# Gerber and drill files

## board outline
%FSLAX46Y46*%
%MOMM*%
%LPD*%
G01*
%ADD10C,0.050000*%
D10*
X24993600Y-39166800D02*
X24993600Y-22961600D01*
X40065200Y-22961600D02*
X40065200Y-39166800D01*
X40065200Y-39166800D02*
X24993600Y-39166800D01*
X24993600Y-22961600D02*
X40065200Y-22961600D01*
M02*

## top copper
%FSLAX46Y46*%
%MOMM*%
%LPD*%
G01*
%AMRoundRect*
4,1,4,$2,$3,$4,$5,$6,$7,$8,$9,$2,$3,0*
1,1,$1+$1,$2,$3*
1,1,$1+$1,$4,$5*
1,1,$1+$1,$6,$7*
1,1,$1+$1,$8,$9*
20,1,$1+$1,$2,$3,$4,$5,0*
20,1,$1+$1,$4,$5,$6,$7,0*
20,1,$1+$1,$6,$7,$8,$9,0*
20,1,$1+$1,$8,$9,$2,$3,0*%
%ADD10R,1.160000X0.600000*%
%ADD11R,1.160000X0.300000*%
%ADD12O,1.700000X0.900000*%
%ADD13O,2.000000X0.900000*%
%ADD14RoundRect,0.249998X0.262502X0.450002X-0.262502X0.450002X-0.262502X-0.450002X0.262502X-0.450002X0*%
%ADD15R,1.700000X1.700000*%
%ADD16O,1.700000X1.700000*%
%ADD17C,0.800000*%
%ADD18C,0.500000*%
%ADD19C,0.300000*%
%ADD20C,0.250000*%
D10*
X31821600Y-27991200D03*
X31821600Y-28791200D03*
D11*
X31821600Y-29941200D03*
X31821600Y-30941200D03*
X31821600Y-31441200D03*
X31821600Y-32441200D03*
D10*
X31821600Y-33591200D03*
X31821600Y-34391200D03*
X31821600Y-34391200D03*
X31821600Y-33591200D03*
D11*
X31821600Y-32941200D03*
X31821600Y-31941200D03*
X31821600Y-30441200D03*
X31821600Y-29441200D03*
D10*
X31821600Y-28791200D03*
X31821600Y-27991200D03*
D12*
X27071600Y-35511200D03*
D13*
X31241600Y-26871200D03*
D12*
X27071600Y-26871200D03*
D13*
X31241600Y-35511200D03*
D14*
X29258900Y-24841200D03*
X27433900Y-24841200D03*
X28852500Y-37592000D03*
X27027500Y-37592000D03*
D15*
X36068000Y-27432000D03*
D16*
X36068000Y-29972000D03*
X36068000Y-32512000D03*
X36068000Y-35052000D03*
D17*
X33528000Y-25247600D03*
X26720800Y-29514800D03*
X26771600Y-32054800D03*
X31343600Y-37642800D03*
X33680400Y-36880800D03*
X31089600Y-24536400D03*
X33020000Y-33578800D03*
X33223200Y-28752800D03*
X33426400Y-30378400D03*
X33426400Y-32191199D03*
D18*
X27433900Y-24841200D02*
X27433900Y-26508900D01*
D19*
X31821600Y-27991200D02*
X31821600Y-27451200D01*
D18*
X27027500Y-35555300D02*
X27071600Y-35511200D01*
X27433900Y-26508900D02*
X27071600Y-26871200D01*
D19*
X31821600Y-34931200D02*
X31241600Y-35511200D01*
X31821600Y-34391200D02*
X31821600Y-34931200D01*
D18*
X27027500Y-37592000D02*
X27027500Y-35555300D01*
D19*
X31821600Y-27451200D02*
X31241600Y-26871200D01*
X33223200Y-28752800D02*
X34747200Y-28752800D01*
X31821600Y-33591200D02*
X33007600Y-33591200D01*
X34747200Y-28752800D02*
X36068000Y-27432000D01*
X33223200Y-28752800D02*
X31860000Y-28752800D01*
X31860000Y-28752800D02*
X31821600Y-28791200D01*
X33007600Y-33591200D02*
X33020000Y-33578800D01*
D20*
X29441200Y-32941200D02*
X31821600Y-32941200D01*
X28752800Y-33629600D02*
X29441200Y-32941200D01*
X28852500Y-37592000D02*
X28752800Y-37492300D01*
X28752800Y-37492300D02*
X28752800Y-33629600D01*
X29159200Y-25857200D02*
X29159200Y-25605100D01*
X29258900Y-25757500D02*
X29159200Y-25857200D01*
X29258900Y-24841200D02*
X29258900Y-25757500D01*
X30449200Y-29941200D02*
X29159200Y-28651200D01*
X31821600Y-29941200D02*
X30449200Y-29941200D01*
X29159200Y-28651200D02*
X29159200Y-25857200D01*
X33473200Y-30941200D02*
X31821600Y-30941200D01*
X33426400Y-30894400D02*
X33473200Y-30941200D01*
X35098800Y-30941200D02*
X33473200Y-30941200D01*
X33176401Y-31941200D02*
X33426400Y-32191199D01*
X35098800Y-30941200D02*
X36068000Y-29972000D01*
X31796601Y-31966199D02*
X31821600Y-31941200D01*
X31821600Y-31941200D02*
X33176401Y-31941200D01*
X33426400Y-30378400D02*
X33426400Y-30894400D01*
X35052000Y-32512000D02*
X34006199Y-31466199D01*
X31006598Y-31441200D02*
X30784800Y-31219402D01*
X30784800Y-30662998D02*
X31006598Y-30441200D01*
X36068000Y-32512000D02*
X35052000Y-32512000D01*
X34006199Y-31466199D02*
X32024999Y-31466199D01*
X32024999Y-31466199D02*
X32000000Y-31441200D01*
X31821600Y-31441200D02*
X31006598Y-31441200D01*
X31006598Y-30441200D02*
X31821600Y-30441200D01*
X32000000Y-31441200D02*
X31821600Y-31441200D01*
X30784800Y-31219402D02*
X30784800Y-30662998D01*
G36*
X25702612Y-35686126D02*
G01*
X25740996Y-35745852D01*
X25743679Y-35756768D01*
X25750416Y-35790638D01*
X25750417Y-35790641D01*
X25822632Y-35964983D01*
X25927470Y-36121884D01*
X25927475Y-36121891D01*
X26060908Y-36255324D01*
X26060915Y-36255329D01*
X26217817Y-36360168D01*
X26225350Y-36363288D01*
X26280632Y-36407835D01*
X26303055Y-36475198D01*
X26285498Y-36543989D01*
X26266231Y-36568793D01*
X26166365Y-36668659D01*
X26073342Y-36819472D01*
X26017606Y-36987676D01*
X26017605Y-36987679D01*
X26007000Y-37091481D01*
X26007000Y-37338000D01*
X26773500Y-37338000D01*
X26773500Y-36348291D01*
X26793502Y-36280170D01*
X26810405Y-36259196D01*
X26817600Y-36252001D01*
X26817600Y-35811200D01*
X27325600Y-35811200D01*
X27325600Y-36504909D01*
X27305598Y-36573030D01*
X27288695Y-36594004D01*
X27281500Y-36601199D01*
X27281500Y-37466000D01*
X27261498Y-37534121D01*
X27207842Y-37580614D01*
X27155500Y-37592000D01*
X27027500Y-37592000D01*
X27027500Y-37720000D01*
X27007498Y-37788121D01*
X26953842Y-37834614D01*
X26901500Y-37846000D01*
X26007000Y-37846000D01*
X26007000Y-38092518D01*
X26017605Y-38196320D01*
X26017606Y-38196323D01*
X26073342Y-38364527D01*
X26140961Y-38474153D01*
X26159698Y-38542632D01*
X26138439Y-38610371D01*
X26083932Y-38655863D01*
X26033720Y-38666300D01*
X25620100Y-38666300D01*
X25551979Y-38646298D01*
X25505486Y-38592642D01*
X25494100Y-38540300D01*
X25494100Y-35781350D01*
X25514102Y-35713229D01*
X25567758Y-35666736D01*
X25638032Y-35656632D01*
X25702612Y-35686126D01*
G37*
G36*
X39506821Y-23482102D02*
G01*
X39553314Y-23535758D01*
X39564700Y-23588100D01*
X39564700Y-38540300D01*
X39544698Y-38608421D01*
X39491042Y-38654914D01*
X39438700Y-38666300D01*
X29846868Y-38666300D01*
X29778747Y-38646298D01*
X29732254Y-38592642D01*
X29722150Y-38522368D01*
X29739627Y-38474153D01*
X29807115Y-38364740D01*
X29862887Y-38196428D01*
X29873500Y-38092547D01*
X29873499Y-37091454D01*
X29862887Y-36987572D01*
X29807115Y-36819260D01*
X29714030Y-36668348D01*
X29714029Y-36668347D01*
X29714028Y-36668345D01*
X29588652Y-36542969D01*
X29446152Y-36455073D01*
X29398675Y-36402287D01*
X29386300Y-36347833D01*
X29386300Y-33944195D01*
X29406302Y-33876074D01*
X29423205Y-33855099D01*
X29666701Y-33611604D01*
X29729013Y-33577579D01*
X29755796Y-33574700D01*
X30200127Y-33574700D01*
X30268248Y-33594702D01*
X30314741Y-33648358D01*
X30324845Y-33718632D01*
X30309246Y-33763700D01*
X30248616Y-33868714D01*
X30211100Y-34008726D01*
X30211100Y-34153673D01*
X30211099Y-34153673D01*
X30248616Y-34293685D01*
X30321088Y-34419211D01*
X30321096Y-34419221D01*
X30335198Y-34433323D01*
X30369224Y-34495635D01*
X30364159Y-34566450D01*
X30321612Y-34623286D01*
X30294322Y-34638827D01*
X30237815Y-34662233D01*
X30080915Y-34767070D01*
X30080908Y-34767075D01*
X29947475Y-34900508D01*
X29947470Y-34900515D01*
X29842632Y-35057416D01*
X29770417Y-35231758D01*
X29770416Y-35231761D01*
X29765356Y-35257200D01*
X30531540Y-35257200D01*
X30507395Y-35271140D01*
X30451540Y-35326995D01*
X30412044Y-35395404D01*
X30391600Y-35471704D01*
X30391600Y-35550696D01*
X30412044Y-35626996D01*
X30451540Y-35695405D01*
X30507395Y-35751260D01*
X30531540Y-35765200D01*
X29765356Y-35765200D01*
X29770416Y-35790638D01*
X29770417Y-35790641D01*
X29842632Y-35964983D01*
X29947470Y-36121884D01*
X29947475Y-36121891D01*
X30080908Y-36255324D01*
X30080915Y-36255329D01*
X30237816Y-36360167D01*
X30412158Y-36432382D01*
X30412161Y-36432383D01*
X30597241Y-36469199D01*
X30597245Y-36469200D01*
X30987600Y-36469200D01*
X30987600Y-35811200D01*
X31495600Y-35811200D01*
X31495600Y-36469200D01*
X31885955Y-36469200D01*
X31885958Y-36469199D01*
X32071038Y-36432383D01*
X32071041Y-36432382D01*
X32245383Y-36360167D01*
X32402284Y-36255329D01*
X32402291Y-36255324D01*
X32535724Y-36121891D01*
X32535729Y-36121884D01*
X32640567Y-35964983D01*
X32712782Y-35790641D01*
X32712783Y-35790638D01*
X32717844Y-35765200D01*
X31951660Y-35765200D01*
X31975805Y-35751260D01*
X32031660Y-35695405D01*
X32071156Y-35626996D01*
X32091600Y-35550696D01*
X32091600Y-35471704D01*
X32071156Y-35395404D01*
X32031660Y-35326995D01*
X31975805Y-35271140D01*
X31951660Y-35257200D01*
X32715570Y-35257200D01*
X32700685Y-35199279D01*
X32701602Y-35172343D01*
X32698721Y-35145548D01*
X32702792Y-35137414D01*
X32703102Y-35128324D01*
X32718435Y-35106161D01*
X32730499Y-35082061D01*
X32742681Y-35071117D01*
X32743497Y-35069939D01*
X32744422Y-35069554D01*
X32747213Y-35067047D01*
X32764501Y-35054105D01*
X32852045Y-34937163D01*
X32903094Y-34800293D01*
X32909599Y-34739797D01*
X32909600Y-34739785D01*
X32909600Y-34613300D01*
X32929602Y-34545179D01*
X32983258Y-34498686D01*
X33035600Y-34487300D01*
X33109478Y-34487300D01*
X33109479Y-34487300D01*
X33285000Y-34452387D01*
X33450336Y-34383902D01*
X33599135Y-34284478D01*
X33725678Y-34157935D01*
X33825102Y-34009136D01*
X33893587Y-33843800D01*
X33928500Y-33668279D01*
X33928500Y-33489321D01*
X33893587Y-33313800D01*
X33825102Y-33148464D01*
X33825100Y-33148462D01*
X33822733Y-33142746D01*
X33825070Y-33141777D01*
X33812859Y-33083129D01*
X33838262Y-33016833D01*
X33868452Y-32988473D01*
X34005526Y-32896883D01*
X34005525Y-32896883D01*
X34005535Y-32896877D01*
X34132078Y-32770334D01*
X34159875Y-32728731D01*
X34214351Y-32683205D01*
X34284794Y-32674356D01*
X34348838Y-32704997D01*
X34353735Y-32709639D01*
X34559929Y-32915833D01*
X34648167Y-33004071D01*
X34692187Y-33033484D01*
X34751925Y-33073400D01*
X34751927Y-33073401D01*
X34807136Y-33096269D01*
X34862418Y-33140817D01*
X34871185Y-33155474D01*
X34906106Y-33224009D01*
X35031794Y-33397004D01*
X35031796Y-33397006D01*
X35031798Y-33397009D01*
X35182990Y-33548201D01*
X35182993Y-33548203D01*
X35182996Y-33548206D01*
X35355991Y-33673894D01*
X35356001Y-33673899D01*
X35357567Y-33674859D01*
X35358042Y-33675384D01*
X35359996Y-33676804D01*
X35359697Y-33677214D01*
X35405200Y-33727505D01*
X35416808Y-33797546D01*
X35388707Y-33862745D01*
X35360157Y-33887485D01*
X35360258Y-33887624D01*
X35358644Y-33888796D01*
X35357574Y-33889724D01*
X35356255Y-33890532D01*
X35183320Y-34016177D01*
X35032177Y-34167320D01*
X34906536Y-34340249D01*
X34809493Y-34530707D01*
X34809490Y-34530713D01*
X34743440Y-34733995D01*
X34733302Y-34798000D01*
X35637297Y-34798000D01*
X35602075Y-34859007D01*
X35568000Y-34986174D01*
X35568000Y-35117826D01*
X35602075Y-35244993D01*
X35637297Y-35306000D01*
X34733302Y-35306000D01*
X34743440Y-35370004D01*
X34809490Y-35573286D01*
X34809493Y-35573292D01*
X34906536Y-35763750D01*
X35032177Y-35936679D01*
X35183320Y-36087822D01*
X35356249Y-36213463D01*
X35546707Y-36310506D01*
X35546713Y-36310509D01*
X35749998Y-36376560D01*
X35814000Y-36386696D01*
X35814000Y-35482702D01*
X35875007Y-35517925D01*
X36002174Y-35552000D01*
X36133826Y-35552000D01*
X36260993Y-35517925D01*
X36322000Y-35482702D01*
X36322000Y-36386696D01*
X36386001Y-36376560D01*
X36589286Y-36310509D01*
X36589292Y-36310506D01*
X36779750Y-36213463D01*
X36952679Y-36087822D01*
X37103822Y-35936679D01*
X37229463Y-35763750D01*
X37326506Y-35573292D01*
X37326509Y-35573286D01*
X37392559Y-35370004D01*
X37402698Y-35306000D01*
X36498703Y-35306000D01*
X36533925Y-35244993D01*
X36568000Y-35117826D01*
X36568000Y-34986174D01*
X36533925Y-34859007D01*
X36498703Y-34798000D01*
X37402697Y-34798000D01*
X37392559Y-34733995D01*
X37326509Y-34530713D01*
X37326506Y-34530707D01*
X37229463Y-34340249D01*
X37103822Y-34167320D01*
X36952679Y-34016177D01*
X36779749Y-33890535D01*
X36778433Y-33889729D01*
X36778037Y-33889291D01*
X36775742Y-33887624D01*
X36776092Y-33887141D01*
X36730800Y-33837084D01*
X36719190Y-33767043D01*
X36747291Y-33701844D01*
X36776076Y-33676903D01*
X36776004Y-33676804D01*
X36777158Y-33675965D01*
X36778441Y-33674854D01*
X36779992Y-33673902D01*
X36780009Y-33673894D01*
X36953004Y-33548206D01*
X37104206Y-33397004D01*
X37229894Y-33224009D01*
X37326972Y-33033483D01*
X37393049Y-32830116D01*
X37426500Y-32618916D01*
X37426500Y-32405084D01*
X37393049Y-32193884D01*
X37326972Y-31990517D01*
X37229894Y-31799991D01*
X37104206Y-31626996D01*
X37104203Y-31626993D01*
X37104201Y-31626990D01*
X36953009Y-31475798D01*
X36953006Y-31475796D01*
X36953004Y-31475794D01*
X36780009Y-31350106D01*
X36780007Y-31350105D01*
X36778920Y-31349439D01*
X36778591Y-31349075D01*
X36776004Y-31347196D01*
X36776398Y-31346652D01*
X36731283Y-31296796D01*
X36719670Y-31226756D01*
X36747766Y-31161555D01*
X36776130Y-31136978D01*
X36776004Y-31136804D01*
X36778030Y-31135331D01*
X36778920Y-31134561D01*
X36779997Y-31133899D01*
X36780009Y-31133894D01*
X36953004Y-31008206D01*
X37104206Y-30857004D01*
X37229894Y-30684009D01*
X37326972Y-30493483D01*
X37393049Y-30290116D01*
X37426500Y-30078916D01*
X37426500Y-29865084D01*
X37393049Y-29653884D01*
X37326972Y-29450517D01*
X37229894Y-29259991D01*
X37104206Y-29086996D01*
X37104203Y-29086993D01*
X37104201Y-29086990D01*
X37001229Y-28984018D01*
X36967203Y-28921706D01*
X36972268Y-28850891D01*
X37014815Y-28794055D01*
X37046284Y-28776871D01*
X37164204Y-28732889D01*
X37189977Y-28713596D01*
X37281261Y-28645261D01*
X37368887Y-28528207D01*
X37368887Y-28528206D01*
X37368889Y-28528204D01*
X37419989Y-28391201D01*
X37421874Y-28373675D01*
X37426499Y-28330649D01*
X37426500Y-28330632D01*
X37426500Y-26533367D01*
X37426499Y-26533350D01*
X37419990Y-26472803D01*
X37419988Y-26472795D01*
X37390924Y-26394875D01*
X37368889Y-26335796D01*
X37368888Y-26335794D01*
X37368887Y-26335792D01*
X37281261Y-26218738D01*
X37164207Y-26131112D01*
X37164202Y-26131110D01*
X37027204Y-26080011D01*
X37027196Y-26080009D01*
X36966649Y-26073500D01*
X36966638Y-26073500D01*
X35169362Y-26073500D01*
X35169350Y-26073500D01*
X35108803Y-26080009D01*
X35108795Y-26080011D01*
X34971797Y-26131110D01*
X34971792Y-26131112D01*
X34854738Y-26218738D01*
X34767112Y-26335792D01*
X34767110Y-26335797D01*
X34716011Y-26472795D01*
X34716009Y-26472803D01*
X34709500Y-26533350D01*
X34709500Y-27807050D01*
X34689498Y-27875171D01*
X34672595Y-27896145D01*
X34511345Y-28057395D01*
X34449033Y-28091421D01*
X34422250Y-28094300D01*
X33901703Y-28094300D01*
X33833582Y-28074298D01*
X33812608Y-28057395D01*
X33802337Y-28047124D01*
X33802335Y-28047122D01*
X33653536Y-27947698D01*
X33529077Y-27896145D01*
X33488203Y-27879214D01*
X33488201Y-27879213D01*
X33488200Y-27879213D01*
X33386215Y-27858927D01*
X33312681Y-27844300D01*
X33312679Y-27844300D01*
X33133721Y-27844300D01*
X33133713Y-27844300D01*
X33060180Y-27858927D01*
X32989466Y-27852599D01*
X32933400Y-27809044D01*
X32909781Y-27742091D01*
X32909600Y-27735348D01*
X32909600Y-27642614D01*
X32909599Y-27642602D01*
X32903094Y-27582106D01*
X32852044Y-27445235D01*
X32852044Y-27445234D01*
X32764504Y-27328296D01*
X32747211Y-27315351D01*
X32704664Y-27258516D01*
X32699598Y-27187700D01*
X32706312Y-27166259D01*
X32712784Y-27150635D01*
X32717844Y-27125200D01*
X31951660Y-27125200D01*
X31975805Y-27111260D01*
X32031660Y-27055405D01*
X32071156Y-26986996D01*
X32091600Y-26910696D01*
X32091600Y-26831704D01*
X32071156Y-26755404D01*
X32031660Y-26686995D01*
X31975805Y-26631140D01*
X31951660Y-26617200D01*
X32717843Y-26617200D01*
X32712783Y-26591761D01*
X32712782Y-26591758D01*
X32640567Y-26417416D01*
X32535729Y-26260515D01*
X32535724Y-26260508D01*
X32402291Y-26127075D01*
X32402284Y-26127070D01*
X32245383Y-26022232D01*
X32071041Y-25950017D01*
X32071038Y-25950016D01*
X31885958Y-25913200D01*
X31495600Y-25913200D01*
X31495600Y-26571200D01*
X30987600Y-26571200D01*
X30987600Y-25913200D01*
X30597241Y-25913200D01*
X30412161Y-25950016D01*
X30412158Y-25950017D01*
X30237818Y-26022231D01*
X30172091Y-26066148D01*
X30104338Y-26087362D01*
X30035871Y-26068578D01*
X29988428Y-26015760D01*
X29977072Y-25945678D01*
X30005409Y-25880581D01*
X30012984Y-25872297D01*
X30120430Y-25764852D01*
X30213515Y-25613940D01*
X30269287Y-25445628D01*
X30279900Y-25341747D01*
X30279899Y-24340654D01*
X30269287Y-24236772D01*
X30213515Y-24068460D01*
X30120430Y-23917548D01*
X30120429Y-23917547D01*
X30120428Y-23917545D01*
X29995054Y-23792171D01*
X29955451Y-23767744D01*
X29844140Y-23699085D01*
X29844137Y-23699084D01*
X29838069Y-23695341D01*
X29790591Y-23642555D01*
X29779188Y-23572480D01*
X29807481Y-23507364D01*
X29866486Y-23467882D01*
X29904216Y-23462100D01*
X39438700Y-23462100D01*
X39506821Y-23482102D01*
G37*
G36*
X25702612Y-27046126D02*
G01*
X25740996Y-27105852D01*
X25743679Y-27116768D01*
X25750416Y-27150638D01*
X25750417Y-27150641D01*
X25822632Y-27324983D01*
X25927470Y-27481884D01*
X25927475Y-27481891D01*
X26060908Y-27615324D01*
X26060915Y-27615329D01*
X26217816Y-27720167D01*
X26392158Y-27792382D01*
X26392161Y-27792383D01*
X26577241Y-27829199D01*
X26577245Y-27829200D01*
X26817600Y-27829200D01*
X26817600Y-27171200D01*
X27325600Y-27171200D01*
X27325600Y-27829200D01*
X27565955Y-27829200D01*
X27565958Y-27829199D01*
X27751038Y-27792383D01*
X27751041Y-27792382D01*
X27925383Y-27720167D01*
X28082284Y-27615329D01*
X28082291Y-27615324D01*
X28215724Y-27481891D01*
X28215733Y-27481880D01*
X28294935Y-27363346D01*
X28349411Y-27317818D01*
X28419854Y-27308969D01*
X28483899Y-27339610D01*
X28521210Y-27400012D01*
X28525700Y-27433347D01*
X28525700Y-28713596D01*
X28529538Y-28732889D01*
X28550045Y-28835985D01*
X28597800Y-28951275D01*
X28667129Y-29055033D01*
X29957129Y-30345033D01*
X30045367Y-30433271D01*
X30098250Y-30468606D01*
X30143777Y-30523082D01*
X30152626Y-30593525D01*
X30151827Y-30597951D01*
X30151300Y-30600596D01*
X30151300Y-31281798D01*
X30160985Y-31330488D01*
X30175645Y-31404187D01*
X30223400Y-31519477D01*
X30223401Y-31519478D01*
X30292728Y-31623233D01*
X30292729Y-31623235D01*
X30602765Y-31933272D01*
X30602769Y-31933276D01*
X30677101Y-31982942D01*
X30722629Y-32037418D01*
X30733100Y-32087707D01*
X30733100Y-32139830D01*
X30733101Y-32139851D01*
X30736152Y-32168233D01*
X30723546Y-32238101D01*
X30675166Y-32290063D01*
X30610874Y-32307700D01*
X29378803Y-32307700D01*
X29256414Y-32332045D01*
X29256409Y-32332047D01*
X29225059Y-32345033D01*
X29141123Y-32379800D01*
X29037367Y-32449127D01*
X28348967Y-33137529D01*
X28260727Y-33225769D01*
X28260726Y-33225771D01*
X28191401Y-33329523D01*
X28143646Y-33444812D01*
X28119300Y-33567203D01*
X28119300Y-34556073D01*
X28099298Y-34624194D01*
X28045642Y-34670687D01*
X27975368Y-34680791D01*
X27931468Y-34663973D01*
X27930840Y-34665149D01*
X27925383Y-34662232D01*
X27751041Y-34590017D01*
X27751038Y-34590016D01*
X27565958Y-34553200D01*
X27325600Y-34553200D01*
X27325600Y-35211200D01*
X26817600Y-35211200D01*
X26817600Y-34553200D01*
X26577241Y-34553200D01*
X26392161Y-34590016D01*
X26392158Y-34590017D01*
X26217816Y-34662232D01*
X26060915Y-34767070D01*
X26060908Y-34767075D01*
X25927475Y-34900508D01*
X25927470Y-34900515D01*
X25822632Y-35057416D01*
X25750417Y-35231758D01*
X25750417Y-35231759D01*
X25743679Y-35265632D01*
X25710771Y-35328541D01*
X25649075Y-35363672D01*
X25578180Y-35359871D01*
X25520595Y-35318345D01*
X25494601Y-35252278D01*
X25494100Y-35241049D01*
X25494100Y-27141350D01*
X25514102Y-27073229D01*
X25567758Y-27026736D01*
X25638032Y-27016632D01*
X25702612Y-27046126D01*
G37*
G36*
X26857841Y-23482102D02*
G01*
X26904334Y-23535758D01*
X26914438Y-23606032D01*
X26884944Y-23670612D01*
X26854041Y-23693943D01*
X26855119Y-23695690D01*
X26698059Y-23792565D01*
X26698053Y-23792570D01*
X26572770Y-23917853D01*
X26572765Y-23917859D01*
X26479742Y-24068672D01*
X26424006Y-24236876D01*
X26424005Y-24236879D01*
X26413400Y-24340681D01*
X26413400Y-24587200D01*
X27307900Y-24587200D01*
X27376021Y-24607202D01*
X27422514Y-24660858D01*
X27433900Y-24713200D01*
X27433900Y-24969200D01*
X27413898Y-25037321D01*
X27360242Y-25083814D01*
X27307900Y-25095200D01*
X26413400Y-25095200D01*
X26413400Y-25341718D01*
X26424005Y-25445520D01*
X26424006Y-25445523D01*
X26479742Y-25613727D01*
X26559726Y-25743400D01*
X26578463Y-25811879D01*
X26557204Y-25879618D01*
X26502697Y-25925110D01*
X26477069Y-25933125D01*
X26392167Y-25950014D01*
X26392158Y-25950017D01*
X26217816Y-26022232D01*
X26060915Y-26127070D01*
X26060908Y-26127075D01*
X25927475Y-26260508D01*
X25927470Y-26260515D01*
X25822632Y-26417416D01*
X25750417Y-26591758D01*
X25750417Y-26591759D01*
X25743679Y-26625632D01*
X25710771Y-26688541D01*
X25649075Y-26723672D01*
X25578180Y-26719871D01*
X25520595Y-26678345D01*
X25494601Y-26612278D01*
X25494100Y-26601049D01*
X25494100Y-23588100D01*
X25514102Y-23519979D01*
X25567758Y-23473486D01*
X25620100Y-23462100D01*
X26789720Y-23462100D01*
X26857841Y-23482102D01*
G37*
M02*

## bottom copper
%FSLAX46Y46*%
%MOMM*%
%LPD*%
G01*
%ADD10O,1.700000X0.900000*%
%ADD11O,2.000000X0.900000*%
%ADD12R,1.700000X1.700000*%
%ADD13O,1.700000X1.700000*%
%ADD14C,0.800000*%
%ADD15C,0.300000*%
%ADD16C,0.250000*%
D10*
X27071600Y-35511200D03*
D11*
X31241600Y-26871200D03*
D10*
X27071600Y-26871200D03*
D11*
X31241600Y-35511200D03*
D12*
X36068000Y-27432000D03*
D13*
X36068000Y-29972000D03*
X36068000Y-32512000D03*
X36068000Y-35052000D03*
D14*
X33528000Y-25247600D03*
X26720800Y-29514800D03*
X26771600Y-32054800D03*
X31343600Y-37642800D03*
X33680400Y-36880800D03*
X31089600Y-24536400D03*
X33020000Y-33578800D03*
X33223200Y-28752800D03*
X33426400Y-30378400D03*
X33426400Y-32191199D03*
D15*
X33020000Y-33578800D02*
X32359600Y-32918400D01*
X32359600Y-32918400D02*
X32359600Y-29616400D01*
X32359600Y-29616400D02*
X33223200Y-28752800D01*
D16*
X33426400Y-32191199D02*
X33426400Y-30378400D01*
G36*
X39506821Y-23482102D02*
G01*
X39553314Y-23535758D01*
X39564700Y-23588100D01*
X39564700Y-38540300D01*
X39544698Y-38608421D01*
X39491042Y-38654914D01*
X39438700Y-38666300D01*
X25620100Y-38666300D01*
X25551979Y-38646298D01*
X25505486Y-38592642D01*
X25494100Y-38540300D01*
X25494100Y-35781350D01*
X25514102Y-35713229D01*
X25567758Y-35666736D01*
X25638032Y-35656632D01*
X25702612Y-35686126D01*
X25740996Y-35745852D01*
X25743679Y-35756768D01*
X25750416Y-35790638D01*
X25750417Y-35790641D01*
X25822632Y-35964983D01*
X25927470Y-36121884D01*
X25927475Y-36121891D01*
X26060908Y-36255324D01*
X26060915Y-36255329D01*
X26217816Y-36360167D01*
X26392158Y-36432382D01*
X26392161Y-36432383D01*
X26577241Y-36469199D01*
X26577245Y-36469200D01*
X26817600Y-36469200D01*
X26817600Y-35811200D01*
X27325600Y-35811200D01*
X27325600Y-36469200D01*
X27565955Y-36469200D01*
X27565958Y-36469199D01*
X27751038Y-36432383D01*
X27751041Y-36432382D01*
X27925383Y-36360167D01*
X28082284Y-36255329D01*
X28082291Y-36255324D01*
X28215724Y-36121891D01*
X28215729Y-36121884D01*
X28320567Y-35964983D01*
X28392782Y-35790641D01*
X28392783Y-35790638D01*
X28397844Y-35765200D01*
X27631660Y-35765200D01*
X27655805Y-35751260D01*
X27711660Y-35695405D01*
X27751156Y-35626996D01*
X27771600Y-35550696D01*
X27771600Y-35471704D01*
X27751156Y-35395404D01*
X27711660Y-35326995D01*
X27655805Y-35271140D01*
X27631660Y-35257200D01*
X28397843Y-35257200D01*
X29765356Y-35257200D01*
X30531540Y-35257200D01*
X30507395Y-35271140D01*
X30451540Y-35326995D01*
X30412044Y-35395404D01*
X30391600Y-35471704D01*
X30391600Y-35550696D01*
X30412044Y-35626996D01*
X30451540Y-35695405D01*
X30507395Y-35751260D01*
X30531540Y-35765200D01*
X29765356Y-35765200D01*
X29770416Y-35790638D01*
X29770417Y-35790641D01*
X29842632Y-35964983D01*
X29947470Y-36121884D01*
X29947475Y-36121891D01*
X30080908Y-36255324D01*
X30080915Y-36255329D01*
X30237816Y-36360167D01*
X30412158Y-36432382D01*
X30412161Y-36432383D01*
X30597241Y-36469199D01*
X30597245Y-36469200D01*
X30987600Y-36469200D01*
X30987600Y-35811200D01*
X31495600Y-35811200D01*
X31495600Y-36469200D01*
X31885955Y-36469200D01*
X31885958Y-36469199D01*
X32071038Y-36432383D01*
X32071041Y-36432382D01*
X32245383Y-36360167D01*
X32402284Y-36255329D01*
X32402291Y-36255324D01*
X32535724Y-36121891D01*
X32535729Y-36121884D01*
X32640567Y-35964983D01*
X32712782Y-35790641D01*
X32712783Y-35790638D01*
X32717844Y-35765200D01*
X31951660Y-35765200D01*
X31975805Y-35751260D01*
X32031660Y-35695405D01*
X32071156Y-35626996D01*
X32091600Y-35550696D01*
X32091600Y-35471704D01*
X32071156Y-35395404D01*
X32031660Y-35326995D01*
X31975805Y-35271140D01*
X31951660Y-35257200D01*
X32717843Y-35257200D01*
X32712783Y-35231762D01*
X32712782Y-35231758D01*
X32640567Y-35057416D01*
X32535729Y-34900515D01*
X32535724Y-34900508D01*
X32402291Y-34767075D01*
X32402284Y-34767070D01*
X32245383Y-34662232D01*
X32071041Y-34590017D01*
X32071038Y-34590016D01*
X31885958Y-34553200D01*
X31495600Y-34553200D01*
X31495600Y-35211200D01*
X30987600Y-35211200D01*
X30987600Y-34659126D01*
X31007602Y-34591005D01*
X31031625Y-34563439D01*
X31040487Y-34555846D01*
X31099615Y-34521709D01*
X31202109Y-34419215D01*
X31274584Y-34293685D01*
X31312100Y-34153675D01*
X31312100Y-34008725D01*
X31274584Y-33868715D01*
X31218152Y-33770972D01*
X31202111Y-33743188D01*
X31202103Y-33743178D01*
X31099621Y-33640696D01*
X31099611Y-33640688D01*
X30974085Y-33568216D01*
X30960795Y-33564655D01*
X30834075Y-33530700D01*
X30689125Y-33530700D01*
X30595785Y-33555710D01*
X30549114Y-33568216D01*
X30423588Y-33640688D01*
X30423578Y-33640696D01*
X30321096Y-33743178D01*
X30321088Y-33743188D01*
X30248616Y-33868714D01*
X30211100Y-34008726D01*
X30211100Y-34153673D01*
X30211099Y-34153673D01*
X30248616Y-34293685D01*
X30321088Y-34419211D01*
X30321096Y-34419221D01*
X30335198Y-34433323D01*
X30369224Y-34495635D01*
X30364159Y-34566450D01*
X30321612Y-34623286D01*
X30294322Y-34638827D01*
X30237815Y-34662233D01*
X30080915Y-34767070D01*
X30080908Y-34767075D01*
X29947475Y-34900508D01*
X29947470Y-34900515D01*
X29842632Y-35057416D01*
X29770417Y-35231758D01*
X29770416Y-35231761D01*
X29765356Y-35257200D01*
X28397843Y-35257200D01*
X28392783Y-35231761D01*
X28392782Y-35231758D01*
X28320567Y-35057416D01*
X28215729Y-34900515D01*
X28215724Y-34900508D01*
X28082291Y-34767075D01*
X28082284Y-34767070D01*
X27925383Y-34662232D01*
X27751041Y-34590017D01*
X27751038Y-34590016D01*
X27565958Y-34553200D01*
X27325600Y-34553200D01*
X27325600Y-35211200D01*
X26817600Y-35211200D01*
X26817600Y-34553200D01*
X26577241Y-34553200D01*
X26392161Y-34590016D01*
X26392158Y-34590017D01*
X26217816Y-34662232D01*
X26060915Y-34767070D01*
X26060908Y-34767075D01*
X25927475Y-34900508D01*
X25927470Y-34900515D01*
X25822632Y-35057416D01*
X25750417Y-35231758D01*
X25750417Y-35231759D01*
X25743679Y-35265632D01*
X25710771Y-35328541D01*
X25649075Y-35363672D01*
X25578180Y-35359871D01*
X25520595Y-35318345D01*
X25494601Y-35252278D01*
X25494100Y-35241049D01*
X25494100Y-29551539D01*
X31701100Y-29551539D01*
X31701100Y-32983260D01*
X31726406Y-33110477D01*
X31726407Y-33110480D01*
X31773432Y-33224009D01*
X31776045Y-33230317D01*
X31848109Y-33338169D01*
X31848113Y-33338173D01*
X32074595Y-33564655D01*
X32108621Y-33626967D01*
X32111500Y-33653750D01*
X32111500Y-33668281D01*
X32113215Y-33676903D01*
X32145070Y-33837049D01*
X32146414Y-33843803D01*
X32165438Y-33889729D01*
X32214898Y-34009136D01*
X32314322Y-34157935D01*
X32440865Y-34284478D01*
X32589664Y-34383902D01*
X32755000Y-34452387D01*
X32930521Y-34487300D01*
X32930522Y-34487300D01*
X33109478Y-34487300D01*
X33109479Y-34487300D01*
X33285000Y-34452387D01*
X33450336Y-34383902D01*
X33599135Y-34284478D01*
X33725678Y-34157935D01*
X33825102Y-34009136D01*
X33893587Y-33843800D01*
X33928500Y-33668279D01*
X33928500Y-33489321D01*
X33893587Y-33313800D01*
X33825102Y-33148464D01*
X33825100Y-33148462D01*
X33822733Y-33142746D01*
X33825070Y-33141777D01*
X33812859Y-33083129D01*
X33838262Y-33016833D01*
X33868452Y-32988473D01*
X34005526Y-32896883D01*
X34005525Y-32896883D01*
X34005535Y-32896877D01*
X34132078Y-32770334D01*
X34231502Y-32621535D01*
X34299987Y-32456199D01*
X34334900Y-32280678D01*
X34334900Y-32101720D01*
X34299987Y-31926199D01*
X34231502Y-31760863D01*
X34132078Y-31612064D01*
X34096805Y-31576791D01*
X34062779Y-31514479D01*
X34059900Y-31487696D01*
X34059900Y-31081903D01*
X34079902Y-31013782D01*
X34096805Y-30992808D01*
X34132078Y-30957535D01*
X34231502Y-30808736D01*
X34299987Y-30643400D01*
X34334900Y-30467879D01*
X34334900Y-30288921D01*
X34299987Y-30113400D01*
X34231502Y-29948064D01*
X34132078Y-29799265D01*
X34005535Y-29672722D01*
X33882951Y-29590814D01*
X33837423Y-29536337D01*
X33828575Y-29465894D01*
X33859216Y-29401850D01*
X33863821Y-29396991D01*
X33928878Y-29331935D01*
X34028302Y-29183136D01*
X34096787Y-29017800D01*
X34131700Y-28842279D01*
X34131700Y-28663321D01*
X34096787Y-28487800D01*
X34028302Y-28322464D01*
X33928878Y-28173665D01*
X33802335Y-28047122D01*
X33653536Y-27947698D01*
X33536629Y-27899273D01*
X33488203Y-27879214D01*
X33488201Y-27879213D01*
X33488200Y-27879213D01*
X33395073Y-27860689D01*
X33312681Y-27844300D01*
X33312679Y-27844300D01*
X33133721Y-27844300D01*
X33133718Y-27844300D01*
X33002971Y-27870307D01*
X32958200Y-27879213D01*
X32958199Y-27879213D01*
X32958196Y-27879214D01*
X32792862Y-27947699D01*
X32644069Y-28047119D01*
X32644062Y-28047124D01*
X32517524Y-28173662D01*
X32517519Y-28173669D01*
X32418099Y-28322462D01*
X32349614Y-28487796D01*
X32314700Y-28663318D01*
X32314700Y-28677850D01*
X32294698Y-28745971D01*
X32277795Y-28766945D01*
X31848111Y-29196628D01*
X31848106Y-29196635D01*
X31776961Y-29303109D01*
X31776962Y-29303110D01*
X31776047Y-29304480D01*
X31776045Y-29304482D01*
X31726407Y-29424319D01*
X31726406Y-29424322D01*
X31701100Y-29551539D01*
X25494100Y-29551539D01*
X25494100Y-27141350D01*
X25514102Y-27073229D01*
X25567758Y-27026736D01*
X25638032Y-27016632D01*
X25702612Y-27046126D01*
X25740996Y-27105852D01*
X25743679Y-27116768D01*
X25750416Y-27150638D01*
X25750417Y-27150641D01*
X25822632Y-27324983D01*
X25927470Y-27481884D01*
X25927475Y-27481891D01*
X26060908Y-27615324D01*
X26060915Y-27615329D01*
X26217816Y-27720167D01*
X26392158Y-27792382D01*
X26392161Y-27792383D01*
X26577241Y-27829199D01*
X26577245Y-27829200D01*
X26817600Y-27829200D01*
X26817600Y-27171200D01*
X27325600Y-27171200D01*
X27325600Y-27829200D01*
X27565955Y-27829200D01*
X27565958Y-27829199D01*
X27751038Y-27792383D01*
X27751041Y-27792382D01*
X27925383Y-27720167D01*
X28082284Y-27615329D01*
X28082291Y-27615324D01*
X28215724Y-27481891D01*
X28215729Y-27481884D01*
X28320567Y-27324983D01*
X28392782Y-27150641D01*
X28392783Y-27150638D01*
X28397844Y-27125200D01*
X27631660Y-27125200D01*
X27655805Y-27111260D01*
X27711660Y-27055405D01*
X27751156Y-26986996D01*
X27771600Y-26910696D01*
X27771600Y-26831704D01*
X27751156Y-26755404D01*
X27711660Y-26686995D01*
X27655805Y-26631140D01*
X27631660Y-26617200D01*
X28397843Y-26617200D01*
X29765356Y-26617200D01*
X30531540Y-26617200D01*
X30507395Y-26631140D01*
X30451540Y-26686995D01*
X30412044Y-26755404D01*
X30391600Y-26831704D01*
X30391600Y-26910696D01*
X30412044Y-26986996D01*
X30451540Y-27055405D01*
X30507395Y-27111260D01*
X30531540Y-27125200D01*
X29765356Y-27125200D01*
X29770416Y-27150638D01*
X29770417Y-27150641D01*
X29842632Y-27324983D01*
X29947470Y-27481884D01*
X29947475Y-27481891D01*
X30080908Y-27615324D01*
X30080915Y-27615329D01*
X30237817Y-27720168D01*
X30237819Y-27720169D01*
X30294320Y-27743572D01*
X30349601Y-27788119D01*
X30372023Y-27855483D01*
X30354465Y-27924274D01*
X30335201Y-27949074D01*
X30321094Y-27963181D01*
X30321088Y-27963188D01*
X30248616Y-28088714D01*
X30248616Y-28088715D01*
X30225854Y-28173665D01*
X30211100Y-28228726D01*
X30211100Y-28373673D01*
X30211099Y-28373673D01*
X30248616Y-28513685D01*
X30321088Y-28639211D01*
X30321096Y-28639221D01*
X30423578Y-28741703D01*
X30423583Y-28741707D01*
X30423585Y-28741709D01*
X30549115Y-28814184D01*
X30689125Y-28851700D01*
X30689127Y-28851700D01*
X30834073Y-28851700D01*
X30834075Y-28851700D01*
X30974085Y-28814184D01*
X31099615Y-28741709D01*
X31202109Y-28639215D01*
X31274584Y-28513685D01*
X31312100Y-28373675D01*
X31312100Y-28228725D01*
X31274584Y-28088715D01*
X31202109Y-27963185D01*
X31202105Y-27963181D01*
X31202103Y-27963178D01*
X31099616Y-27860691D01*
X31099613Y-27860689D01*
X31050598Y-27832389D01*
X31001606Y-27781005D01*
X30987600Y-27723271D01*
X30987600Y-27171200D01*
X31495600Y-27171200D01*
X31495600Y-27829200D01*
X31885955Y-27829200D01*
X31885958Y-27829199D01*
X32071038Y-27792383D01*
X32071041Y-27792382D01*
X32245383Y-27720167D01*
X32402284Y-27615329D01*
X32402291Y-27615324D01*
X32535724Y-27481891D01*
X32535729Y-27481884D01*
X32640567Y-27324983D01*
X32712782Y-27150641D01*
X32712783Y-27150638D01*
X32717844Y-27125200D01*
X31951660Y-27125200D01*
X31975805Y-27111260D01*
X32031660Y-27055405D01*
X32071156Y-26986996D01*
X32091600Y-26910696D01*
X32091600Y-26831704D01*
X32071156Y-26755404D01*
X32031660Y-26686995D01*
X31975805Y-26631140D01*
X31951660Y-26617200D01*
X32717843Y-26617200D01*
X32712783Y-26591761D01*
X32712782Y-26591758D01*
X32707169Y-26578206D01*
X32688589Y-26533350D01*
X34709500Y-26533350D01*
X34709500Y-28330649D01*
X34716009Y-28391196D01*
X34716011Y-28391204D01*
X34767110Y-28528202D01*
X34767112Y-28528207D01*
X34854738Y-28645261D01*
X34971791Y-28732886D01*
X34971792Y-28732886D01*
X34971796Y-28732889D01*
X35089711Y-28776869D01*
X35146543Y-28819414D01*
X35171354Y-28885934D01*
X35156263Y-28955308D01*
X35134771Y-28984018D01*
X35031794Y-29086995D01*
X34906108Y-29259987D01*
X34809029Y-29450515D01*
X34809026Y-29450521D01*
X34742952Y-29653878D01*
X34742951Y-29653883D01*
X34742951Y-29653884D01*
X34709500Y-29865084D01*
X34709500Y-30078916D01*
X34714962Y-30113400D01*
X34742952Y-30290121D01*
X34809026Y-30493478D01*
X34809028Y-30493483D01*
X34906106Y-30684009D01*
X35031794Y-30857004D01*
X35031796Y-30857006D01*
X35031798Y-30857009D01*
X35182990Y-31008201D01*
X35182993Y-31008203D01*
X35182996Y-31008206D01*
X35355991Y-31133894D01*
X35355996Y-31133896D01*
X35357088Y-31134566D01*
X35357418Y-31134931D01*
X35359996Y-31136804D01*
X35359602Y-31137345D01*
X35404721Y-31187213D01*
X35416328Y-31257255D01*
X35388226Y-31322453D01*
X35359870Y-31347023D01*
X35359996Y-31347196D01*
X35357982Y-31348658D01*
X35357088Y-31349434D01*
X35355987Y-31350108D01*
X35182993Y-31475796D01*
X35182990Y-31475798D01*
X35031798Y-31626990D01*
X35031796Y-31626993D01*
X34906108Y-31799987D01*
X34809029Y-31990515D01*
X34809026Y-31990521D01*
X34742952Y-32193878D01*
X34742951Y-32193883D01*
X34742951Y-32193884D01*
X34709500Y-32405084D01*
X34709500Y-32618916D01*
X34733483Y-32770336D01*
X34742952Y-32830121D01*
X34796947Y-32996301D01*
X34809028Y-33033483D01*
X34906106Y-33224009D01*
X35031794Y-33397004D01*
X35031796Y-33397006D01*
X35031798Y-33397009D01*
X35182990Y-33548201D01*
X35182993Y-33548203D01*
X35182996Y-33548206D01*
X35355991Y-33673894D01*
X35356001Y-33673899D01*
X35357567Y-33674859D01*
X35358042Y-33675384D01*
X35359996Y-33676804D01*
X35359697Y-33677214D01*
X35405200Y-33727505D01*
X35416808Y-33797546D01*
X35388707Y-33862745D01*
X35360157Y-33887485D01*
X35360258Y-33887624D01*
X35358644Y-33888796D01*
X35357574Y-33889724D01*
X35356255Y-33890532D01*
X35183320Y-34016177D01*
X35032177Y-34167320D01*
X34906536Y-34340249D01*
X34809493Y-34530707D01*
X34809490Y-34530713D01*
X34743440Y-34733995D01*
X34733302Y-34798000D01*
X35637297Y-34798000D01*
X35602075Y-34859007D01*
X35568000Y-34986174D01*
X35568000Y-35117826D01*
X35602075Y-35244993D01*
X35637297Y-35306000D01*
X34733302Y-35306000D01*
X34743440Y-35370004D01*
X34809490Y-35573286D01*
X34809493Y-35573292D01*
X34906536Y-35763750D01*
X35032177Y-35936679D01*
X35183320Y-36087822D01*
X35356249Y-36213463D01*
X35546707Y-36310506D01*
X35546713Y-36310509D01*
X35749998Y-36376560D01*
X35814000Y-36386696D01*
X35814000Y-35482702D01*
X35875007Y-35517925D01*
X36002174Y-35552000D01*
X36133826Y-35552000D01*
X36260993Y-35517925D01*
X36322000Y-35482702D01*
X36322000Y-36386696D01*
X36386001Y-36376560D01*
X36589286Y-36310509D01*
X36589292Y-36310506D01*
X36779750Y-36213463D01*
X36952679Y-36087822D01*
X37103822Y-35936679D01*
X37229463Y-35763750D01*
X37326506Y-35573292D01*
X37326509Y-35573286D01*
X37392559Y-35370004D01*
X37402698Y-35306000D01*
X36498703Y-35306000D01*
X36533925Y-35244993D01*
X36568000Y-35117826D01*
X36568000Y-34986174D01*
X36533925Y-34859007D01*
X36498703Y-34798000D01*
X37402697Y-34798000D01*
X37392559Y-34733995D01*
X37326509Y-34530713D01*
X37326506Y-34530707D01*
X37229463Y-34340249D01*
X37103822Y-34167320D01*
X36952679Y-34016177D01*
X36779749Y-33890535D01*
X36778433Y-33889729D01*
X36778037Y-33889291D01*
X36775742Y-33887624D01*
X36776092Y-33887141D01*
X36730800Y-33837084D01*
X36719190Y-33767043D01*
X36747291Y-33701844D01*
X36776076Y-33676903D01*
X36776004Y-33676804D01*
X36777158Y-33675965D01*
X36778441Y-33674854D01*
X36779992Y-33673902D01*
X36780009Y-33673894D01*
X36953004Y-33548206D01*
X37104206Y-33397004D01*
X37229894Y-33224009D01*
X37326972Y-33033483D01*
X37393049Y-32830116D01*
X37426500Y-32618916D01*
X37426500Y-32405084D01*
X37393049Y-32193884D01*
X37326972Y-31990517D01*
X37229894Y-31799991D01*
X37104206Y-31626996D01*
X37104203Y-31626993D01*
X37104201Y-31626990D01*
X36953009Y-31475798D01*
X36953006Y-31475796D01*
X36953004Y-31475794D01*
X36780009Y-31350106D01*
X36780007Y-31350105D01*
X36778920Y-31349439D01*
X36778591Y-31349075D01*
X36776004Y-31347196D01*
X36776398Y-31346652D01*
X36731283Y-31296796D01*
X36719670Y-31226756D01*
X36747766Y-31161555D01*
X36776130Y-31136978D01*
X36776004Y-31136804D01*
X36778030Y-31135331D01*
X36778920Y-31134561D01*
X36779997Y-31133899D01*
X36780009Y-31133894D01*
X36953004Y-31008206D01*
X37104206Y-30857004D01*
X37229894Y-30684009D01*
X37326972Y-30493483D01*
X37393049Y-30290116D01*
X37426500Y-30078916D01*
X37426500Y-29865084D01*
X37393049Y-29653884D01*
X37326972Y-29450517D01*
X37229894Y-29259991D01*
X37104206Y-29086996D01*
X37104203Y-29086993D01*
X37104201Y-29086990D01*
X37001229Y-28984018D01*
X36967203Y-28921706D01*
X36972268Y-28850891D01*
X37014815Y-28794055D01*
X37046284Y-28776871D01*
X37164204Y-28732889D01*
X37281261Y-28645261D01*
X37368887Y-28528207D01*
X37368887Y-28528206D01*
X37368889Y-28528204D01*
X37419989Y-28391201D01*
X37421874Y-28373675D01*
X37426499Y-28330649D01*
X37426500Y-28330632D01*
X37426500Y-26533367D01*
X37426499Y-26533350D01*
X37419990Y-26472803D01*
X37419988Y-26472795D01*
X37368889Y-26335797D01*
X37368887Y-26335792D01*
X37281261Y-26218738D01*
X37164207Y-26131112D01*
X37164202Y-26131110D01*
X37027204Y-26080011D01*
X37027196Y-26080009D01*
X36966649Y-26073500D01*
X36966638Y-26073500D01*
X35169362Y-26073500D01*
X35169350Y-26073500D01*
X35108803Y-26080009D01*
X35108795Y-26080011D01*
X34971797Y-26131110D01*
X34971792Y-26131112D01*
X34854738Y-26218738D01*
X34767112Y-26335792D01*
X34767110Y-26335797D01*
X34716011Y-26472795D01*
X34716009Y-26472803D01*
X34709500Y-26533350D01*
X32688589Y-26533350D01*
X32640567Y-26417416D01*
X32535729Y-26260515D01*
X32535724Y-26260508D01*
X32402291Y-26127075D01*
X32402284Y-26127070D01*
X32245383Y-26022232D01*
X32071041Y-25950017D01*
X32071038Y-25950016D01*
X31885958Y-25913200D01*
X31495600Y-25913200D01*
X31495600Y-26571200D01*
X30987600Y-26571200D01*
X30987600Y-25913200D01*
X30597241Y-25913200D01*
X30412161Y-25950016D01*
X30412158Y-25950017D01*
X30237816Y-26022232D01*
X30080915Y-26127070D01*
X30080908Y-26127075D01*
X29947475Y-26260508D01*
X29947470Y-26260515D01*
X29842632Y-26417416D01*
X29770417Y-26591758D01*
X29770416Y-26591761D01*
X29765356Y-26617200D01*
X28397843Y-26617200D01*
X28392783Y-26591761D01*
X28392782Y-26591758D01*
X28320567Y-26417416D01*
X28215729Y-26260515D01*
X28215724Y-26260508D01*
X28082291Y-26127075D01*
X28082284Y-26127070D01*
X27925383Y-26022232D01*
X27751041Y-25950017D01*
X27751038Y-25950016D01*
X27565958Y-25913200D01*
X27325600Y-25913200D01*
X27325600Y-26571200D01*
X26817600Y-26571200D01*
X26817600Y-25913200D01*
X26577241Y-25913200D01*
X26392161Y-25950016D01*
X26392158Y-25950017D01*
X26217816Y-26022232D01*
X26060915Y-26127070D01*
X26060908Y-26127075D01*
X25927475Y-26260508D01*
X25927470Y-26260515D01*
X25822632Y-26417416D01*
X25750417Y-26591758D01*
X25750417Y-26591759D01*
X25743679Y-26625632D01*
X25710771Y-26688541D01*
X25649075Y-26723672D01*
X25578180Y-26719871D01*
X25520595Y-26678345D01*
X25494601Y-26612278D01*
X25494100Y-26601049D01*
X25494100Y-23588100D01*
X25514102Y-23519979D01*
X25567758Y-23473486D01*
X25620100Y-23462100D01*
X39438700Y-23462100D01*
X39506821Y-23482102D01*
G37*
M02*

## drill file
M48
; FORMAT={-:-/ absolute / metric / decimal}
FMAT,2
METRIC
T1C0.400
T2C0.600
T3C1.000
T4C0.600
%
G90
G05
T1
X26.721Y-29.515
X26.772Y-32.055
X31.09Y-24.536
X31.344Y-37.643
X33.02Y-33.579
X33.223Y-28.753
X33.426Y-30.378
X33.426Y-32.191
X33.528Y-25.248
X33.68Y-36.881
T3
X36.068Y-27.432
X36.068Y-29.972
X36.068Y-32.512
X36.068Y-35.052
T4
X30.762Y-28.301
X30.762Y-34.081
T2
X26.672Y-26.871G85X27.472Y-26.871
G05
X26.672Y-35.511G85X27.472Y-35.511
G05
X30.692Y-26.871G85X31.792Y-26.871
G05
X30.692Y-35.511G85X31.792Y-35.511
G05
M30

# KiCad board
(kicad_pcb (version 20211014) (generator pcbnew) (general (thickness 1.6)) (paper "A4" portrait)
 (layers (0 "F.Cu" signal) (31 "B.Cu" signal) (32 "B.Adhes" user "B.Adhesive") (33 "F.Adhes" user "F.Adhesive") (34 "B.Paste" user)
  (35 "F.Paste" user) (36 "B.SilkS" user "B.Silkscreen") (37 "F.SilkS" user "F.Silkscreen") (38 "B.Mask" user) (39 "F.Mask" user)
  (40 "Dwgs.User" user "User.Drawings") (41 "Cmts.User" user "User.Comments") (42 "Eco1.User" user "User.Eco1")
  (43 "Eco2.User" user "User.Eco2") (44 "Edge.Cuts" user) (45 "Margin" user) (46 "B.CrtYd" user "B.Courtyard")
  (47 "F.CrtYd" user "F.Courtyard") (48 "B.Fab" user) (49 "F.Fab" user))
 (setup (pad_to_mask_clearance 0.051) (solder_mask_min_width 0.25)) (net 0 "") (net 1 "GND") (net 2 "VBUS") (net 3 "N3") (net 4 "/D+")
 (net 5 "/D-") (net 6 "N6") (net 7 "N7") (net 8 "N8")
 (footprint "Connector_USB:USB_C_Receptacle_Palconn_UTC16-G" (layer "F.Cu") (at 29.3116 31.1912 -90)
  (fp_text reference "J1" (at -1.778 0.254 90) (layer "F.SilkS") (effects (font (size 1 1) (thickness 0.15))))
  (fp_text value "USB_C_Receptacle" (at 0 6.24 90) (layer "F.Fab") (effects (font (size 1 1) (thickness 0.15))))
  (pad "" np_thru_hole circle locked (at -2.89 -1.45 90) (size 0.6 0.6) (drill 0.6) (layers *.Cu *.Mask))
  (pad "" np_thru_hole circle locked (at 2.89 -1.45 90) (size 0.6 0.6) (drill 0.6) (layers *.Cu *.Mask))
  (pad "A1" smd rect locked (at -3.2 -2.51 270) (size 0.6 1.16) (layers "F.Cu" "F.Paste" "F.Mask") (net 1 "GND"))
  (pad "A4" smd rect locked (at -2.4 -2.51 270) (size 0.6 1.16) (layers "F.Cu" "F.Paste" "F.Mask") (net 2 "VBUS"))
  (pad "A5" smd rect locked (at -1.25 -2.51 90) (size 0.3 1.16) (layers "F.Cu" "F.Paste" "F.Mask") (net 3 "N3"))
  (pad "A6" smd rect locked (at -0.25 -2.51 90) (size 0.3 1.16) (layers "F.Cu" "F.Paste" "F.Mask") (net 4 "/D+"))
  (pad "A7" smd rect locked (at 0.25 -2.51 90) (size 0.3 1.16) (layers "F.Cu" "F.Paste" "F.Mask") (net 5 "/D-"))
  (pad "A8" smd rect locked (at 1.25 -2.51 90) (size 0.3 1.16) (layers "F.Cu" "F.Paste" "F.Mask") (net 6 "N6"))
  (pad "A9" smd rect locked (at 2.4 -2.51 270) (size 0.6 1.16) (layers "F.Cu" "F.Paste" "F.Mask") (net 2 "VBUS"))
  (pad "A12" smd rect locked (at 3.2 -2.51 270) (size 0.6 1.16) (layers "F.Cu" "F.Paste" "F.Mask") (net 1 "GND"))
  (pad "B1" smd rect locked (at 3.2 -2.51 270) (size 0.6 1.16) (layers "F.Cu" "F.Paste" "F.Mask") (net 1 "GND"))
  (pad "B4" smd rect locked (at 2.4 -2.51 270) (size 0.6 1.16) (layers "F.Cu" "F.Paste" "F.Mask") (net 2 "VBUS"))
  (pad "B5" smd rect locked (at 1.75 -2.51 90) (size 0.3 1.16) (layers "F.Cu" "F.Paste" "F.Mask") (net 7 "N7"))
  (pad "B6" smd rect locked (at 0.75 -2.51 90) (size 0.3 1.16) (layers "F.Cu" "F.Paste" "F.Mask") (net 4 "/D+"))
  (pad "B7" smd rect locked (at -0.75 -2.51 90) (size 0.3 1.16) (layers "F.Cu" "F.Paste" "F.Mask") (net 5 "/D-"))
  (pad "B8" smd rect locked (at -1.75 -2.51 90) (size 0.3 1.16) (layers "F.Cu" "F.Paste" "F.Mask") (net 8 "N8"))
  (pad "B9" smd rect locked (at -2.4 -2.51 270) (size 0.6 1.16) (layers "F.Cu" "F.Paste" "F.Mask") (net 2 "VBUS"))
  (pad "B12" smd rect locked (at -3.2 -2.51 270) (size 0.6 1.16) (layers "F.Cu" "F.Paste" "F.Mask") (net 1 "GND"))
  (pad "S1" thru_hole oval locked (at 4.32 2.24) (size 1.7 0.9) (drill oval 1.4 0.6) (layers *.Cu *.Mask) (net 1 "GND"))
  (pad "S1" thru_hole oval locked (at -4.32 -1.93) (size 2 0.9) (drill oval 1.7 0.6) (layers *.Cu *.Mask) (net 1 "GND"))
  (pad "S1" thru_hole oval locked (at -4.32 2.24) (size 1.7 0.9) (drill oval 1.4 0.6) (layers *.Cu *.Mask) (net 1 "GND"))
  (pad "S1" thru_hole oval locked (at 4.32 -1.93) (size 2 0.9) (drill oval 1.7 0.6) (layers *.Cu *.Mask) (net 1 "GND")))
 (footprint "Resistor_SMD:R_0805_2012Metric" (layer "F.Cu") (at 28.3464 24.8412 180)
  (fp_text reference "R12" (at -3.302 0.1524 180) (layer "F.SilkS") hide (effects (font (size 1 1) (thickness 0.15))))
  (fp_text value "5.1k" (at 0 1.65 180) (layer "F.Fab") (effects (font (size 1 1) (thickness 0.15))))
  (pad "1" smd roundrect locked (at -0.9125 0 180) (size 1.025 1.4) (layers "F.Cu" "F.Paste" "F.Mask") (roundrect_rratio 0.2439004878)
   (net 3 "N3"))
  (pad "2" smd roundrect locked (at 0.9125 0 180) (size 1.025 1.4) (layers "F.Cu" "F.Paste" "F.Mask") (roundrect_rratio 0.2439004878)
   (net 1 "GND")))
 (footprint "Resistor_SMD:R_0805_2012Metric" (layer "F.Cu") (at 27.94 37.592 180)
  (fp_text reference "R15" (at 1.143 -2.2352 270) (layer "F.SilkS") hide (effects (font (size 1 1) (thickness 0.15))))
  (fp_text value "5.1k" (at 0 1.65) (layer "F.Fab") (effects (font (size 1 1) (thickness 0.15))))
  (pad "1" smd roundrect locked (at -0.9125 0 180) (size 1.025 1.4) (layers "F.Cu" "F.Paste" "F.Mask") (roundrect_rratio 0.2439004878)
   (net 7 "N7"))
  (pad "2" smd roundrect locked (at 0.9125 0 180) (size 1.025 1.4) (layers "F.Cu" "F.Paste" "F.Mask") (roundrect_rratio 0.2439004878)
   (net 1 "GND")))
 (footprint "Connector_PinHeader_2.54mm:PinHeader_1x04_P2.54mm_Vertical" (layer "F.Cu") (at 36.068 27.432)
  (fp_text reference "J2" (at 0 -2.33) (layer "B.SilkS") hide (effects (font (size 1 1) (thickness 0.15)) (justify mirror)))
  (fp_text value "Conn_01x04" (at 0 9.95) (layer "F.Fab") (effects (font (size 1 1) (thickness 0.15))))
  (pad "1" thru_hole rect locked (at 0 0) (size 1.7 1.7) (drill 1) (layers *.Cu *.Mask) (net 2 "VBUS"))
  (pad "2" thru_hole oval locked (at 0 2.54) (size 1.7 1.7) (drill 1) (layers *.Cu *.Mask) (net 4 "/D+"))
  (pad "3" thru_hole oval locked (at 0 5.08) (size 1.7 1.7) (drill 1) (layers *.Cu *.Mask) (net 5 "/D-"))
  (pad "4" thru_hole oval locked (at 0 7.62) (size 1.7 1.7) (drill 1) (layers *.Cu *.Mask) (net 1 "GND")))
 (gr_line (start 24.9936 39.1668) (end 24.9936 22.9616) (layer "Edge.Cuts") (width 0.05))
 (gr_line (start 40.0652 22.9616) (end 40.0652 39.1668) (layer "Edge.Cuts") (width 0.05))
 (gr_line (start 40.0652 39.1668) (end 24.9936 39.1668) (layer "Edge.Cuts") (width 0.05))
 (gr_line (start 24.9936 22.9616) (end 40.0652 22.9616) (layer "Edge.Cuts") (width 0.05))
 (segment (start 27.4339 24.8412) (end 27.4339 26.5089) (width 0.5) (layer "F.Cu") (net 1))
 (segment (start 31.8216 27.9912) (end 31.8216 27.4512) (width 0.3) (layer "F.Cu") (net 1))
 (segment (start 27.0275 35.5553) (end 27.0716 35.5112) (width 0.5) (layer "F.Cu") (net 1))
 (segment (start 27.4339 26.5089) (end 27.0716 26.8712) (width 0.5) (layer "F.Cu") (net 1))
 (segment (start 31.8216 34.9312) (end 31.2416 35.5112) (width 0.3) (layer "F.Cu") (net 1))
 (segment (start 31.8216 34.3912) (end 31.8216 34.9312) (width 0.3) (layer "F.Cu") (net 1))
 (segment (start 27.0275 37.592) (end 27.0275 35.5553) (width 0.5) (layer "F.Cu") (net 1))
 (segment (start 31.8216 27.4512) (end 31.2416 26.8712) (width 0.3) (layer "F.Cu") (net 1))
 (via (at 33.528 25.2476) (size 0.8) (drill 0.4) (layers "F.Cu" "B.Cu") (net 1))
 (via (at 26.7208 29.5148) (size 0.8) (drill 0.4) (layers "F.Cu" "B.Cu") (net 1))
 (via (at 26.7716 32.0548) (size 0.8) (drill 0.4) (layers "F.Cu" "B.Cu") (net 1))
 (via (at 31.3436 37.6428) (size 0.8) (drill 0.4) (layers "F.Cu" "B.Cu") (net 1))
 (via (at 33.6804 36.8808) (size 0.8) (drill 0.4) (layers "F.Cu" "B.Cu") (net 1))
 (via (at 31.0896 24.5364) (size 0.8) (drill 0.4) (layers "F.Cu" "B.Cu") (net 1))
 (segment (start 33.2232 28.7528) (end 34.7472 28.7528) (width 0.3) (layer "F.Cu") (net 2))
 (segment (start 31.8216 33.5912) (end 33.0076 33.5912) (width 0.3) (layer "F.Cu") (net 2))
 (segment (start 34.7472 28.7528) (end 36.068 27.432) (width 0.3) (layer "F.Cu") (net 2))
 (segment (start 33.2232 28.7528) (end 31.86 28.7528) (width 0.3) (layer "F.Cu") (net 2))
 (segment (start 31.86 28.7528) (end 31.8216 28.7912) (width 0.3) (layer "F.Cu") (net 2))
 (segment (start 33.0076 33.5912) (end 33.02 33.5788) (width 0.3) (layer "F.Cu") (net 2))
 (via (at 33.02 33.5788) (size 0.8) (drill 0.4) (layers "F.Cu" "B.Cu") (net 2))
 (via (at 33.2232 28.7528) (size 0.8) (drill 0.4) (layers "F.Cu" "B.Cu") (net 2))
 (segment (start 33.02 33.5788) (end 32.3596 32.9184) (width 0.3) (layer "B.Cu") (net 2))
 (segment (start 32.3596 32.9184) (end 32.3596 29.6164) (width 0.3) (layer "B.Cu") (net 2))
 (segment (start 32.3596 29.6164) (end 33.2232 28.7528) (width 0.3) (layer "B.Cu") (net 2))
 (segment (start 29.4412 32.9412) (end 31.8216 32.9412) (width 0.25) (layer "F.Cu") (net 7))
 (segment (start 28.7528 33.6296) (end 29.4412 32.9412) (width 0.25) (layer "F.Cu") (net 7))
 (segment (start 28.8525 37.592) (end 28.7528 37.4923) (width 0.25) (layer "F.Cu") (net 7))
 (segment (start 28.7528 37.4923) (end 28.7528 33.6296) (width 0.25) (layer "F.Cu") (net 7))
 (segment (start 29.1592 25.8572) (end 29.1592 25.6051) (width 0.25) (layer "F.Cu") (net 3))
 (segment (start 29.2589 25.7575) (end 29.1592 25.8572) (width 0.25) (layer "F.Cu") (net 3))
 (segment (start 29.2589 24.8412) (end 29.2589 25.7575) (width 0.25) (layer "F.Cu") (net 3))
 (segment (start 30.4492 29.9412) (end 29.1592 28.6512) (width 0.25) (layer "F.Cu") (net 3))
 (segment (start 31.8216 29.9412) (end 30.4492 29.9412) (width 0.25) (layer "F.Cu") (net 3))
 (segment (start 29.1592 28.6512) (end 29.1592 25.8572) (width 0.25) (layer "F.Cu") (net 3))
 (segment (start 33.4732 30.9412) (end 31.8216 30.9412) (width 0.25) (layer "F.Cu") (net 4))
 (segment (start 33.4264 30.8944) (end 33.4732 30.9412) (width 0.25) (layer "F.Cu") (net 4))
 (segment (start 35.0988 30.9412) (end 33.4732 30.9412) (width 0.25) (layer "F.Cu") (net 4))
 (segment (start 33.176401 31.9412) (end 33.4264 32.191199) (width 0.25) (layer "F.Cu") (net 4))
 (segment (start 35.0988 30.9412) (end 36.068 29.972) (width 0.25) (layer "F.Cu") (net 4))
 (segment (start 31.796601 31.966199) (end 31.8216 31.9412) (width 0.25) (layer "F.Cu") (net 4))
 (segment (start 31.8216 31.9412) (end 33.176401 31.9412) (width 0.25) (layer "F.Cu") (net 4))
 (segment (start 33.4264 30.3784) (end 33.4264 30.8944) (width 0.25) (layer "F.Cu") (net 4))
 (via (at 33.4264 30.3784) (size 0.8) (drill 0.4) (layers "F.Cu" "B.Cu") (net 4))
 (via (at 33.4264 32.191199) (size 0.8) (drill 0.4) (layers "F.Cu" "B.Cu") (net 4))
 (segment (start 33.4264 32.191199) (end 33.4264 30.3784) (width 0.25) (layer "B.Cu") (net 4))
 (segment (start 35.052 32.512) (end 34.006199 31.466199) (width 0.25) (layer "F.Cu") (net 5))
 (segment (start 31.006598 31.4412) (end 30.7848 31.219402) (width 0.25) (layer "F.Cu") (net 5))
 (segment (start 30.7848 30.662998) (end 31.006598 30.4412) (width 0.25) (layer "F.Cu") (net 5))
 (segment (start 36.068 32.512) (end 35.052 32.512) (width 0.25) (layer "F.Cu") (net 5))
 (segment (start 34.006199 31.466199) (end 32.024999 31.466199) (width 0.25) (layer "F.Cu") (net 5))
 (segment (start 32.024999 31.466199) (end 32 31.4412) (width 0.25) (layer "F.Cu") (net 5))
 (segment (start 31.8216 31.4412) (end 31.006598 31.4412) (width 0.25) (layer "F.Cu") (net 5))
 (segment (start 31.006598 30.4412) (end 31.8216 30.4412) (width 0.25) (layer "F.Cu") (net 5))
 (segment (start 32 31.4412) (end 31.8216 31.4412) (width 0.25) (layer "F.Cu") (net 5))
 (segment (start 30.7848 31.219402) (end 30.7848 30.662998) (width 0.25) (layer "F.Cu") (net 5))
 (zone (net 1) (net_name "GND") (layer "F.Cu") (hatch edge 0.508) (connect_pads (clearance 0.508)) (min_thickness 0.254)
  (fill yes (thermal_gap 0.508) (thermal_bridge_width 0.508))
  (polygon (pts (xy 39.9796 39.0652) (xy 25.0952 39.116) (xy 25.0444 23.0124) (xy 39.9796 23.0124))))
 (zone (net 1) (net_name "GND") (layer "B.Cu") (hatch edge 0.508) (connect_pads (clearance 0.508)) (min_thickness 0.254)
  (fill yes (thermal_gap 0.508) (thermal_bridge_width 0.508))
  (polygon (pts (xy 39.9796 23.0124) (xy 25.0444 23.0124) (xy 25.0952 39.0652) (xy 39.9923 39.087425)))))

